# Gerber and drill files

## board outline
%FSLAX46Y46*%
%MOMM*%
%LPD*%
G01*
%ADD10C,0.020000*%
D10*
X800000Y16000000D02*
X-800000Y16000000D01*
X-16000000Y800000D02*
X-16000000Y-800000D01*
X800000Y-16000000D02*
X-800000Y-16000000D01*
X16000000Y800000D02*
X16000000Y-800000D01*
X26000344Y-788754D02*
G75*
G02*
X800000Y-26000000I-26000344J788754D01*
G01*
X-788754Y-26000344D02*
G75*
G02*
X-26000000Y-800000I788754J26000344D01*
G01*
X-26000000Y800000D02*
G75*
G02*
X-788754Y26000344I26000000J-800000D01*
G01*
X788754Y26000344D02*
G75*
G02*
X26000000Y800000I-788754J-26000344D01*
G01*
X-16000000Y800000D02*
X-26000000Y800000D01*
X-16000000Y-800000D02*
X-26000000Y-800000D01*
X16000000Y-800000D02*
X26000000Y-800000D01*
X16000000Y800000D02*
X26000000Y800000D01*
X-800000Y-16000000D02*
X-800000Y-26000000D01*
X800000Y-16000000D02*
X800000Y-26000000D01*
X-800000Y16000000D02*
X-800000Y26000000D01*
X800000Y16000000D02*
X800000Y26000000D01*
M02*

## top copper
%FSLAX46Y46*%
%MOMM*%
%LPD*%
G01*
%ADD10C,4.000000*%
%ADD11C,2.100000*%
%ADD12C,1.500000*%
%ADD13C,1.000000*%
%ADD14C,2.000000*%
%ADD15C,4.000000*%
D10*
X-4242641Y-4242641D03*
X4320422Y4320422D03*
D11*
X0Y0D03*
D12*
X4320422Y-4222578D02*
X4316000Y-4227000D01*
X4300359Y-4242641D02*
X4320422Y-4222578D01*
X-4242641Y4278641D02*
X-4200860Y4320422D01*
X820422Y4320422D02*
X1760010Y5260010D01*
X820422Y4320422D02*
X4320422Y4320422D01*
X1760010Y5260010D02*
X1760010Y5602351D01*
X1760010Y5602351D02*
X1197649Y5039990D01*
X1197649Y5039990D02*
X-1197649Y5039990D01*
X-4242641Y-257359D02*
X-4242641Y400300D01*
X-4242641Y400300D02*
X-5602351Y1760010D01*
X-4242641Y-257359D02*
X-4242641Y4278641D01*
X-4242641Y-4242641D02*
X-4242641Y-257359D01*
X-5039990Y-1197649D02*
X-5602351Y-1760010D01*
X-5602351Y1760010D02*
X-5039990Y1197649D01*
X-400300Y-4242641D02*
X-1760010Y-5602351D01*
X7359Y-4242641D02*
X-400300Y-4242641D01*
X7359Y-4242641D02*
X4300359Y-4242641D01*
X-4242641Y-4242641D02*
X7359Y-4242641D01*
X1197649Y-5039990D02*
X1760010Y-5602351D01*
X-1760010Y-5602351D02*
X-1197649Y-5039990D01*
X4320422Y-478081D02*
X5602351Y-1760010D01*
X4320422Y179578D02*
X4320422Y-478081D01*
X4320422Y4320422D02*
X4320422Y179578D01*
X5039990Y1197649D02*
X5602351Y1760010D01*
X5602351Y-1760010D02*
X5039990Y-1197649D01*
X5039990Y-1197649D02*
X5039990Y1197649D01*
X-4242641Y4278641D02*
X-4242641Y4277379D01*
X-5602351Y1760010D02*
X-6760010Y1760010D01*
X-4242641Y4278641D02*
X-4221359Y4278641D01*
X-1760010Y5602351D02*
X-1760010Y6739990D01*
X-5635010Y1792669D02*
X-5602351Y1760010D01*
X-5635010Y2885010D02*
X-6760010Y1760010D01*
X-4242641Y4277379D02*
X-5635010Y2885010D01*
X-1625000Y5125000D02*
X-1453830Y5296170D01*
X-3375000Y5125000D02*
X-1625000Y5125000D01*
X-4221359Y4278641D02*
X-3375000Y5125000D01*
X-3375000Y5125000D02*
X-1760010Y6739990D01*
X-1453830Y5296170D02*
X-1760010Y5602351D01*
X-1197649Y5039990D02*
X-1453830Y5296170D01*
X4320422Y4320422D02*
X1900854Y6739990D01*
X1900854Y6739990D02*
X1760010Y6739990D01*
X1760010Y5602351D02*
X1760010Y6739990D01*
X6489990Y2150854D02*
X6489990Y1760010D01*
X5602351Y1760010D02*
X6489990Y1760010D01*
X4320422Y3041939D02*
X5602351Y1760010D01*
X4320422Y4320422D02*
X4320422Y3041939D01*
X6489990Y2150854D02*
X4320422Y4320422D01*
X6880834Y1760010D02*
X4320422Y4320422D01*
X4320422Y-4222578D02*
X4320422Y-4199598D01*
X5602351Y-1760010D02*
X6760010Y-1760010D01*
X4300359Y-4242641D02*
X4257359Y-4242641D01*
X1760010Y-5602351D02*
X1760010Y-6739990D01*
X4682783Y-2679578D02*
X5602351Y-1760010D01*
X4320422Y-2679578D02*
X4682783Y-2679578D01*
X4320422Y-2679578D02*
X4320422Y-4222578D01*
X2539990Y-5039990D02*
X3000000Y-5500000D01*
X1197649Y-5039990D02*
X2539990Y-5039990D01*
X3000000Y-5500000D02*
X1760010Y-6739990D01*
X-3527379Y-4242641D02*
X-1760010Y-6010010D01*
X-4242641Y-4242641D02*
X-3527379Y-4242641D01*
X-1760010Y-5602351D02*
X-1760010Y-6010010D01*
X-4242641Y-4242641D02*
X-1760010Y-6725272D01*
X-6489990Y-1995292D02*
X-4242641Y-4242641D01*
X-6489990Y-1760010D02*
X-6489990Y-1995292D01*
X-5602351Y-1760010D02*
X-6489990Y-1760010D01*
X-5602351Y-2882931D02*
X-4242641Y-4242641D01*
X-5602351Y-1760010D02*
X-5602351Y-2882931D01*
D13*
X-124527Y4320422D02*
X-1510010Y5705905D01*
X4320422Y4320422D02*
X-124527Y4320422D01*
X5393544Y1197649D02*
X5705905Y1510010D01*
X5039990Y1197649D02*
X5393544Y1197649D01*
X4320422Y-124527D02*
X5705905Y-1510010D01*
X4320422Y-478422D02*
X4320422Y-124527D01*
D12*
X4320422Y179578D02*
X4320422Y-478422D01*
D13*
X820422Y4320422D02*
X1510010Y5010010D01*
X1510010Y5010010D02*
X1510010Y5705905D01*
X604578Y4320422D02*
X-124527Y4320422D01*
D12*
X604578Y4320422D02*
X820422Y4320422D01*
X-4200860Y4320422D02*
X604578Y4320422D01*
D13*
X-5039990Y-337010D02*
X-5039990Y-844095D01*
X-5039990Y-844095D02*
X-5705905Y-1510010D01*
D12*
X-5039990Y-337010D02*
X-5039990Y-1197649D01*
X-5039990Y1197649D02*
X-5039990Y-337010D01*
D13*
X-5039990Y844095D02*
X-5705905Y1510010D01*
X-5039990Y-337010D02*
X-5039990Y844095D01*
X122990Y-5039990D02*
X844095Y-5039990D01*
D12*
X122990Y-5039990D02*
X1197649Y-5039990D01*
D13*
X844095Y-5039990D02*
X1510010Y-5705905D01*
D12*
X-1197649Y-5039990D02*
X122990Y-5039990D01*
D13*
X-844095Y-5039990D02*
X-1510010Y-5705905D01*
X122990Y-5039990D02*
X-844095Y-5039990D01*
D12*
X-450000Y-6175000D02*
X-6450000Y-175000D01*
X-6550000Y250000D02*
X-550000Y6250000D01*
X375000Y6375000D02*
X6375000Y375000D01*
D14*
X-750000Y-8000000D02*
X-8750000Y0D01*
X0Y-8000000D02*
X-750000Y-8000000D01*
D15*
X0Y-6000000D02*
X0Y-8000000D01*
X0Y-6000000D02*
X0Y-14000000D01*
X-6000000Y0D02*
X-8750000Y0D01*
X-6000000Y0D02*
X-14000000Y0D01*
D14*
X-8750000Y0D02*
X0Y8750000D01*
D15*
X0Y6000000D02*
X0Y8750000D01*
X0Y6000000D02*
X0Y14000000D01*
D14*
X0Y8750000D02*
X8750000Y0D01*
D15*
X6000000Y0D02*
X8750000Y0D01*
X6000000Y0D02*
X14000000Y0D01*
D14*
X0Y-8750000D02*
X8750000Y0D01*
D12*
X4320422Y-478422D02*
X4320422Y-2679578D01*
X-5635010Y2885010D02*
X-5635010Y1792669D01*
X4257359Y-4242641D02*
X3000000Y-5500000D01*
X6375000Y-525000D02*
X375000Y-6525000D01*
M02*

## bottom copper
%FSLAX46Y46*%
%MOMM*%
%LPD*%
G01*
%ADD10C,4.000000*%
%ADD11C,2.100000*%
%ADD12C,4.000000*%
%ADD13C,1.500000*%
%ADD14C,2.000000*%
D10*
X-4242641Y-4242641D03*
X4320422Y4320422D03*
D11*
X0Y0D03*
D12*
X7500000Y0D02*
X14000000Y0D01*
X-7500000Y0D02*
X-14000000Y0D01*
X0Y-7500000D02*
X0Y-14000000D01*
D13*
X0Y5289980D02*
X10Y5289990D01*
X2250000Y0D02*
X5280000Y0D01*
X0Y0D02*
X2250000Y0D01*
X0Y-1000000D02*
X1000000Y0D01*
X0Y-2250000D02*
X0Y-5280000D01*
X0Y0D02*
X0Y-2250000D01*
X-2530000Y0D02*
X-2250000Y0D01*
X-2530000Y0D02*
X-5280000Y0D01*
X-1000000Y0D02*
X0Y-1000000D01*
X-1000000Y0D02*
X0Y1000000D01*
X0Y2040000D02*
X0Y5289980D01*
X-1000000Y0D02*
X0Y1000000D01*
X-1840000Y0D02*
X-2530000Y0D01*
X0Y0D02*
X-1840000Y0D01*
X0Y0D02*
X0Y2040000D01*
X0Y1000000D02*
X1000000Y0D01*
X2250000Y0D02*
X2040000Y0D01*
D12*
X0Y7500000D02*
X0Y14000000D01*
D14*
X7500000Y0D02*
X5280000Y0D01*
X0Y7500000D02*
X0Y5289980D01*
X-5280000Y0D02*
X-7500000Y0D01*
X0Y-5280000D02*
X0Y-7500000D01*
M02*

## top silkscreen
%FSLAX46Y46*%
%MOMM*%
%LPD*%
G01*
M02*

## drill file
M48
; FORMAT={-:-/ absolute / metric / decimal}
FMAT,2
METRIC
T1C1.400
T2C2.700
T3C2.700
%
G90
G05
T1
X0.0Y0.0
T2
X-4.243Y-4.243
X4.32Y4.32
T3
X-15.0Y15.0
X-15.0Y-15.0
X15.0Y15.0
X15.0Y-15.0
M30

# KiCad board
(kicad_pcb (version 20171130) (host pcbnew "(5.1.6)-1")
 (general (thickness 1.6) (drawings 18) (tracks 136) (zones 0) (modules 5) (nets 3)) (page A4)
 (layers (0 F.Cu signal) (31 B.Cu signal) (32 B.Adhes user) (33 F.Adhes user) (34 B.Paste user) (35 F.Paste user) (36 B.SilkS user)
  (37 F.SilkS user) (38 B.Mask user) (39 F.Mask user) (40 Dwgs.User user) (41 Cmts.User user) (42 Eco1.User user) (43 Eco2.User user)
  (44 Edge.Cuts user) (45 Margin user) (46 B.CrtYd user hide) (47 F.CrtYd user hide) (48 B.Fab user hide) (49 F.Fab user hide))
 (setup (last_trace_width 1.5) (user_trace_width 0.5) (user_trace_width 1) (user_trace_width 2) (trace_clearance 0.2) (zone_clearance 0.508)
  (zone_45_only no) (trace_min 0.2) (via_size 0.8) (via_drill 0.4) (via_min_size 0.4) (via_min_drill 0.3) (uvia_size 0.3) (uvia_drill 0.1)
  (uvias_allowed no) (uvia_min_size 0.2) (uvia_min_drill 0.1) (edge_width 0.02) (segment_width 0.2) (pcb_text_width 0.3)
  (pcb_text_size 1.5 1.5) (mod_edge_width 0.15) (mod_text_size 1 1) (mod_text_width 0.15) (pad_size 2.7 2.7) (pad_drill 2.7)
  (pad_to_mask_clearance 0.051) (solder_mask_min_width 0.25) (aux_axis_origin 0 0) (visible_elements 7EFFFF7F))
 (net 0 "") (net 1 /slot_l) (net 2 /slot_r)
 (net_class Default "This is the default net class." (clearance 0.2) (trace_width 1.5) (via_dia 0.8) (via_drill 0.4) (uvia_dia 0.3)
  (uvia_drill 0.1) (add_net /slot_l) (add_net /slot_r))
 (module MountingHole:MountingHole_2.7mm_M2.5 (layer F.Cu) (at -15 -15 90)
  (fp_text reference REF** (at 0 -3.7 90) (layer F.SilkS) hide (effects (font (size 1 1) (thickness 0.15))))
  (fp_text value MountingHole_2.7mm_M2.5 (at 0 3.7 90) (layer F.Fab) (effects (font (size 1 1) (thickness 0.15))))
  (pad 1 np_thru_hole circle (at 0 0 90) (size 2.7 2.7) (drill 2.7) (layers *.Cu *.Mask)))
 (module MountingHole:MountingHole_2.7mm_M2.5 (layer F.Cu) (at 15 -15)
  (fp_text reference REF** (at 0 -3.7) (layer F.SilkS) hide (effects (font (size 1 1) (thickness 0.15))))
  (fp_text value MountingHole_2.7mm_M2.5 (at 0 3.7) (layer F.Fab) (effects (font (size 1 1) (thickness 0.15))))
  (pad 1 np_thru_hole circle (at 0 0) (size 2.7 2.7) (drill 2.7) (layers *.Cu *.Mask)))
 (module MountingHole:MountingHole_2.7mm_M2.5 (layer F.Cu) (at 15 15)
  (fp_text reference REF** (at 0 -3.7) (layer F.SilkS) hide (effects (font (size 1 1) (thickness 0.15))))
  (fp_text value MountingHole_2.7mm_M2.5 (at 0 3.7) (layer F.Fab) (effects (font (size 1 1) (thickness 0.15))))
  (pad 1 np_thru_hole circle (at 0 0) (size 2.7 2.7) (drill 2.7) (layers *.Cu *.Mask)))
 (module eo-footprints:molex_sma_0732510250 (layer F.Cu) (at 0 0 45)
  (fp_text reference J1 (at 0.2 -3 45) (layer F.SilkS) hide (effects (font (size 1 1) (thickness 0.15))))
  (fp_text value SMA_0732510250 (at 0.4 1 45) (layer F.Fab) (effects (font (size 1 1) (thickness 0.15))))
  (pad 2 thru_hole circle (at -6 0 45) (size 4 4) (drill 2.7) (layers *.Cu *.Mask) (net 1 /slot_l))
  (pad 2 thru_hole circle (at 6.11 0 45) (size 4 4) (drill 2.7) (layers *.Cu *.Mask) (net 1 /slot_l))
  (pad 1 thru_hole circle (at 0 0 45) (size 2.1 2.1) (drill 1.4) (layers *.Cu *.Mask) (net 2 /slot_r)))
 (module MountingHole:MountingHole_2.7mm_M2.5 (layer F.Cu) (at -15 15)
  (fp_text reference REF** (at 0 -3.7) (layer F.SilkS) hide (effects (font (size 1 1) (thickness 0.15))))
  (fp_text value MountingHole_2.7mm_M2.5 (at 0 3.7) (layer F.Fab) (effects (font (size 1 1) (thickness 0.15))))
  (pad 1 np_thru_hole circle (at 0 0) (size 2.7 2.7) (drill 2.7) (layers *.Cu *.Mask)))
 (gr_line (start 0.8 -16) (end -0.8 -16) (layer Edge.Cuts) (width 0.02))
 (gr_line (start -16 -0.8) (end -16 0.8) (layer Edge.Cuts) (width 0.02))
 (gr_line (start 0.8 16) (end -0.8 16) (layer Edge.Cuts) (width 0.02))
 (gr_line (start 16 -0.8) (end 16 0.8) (layer Edge.Cuts) (width 0.02))
 (gr_arc (start 0 0) (end 0.8 26) (angle -86.5) (layer Edge.Cuts) (width 0.02))
 (gr_arc (start 0 0) (end -26 0.8) (angle -86.5) (layer Edge.Cuts) (width 0.02))
 (gr_arc (start 0 0) (end -26 -0.8) (angle 86.5) (layer Edge.Cuts) (width 0.02))
 (gr_arc (start 0 0) (end 26 -0.8) (angle -86.5) (layer Edge.Cuts) (width 0.02))
 (gr_line (start -16 -0.8) (end -26 -0.8) (layer Edge.Cuts) (width 0.02))
 (gr_line (start -16 0.8) (end -26 0.8) (layer Edge.Cuts) (width 0.02))
 (gr_line (start 16 0.8) (end 26 0.8) (layer Edge.Cuts) (width 0.02))
 (gr_line (start 16 -0.8) (end 26 -0.8) (layer Edge.Cuts) (width 0.02))
 (gr_line (start -0.8 16) (end -0.8 26) (layer Edge.Cuts) (width 0.02))
 (gr_line (start 0.8 16) (end 0.8 26) (layer Edge.Cuts) (width 0.02))
 (gr_line (start -0.8 -16) (end -0.8 -26) (layer Edge.Cuts) (width 0.02))
 (gr_line (start 0.8 -16) (end 0.8 -26) (layer Edge.Cuts) (width 0.02))
 (segment (start 7.5 0) (end 14 0) (width 4) (layer B.Cu) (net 2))
 (segment (start -7.5 0) (end -14 0) (width 4) (layer B.Cu) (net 2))
 (segment (start 0 7.5) (end 0 14) (width 4) (layer B.Cu) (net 2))
 (segment (start 0 -5.28998) (end 0.00001 -5.28999) (width 1.5) (layer B.Cu) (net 2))
 (segment (start 2.25 0) (end 5.28 0) (width 1.5) (layer B.Cu) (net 2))
 (segment (start 0 0) (end 2.25 0) (width 1.5) (layer B.Cu) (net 2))
 (segment (start 0 1) (end 1 0) (width 1.5) (layer B.Cu) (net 2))
 (segment (start 0 2.25) (end 0 5.28) (width 1.5) (layer B.Cu) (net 2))
 (segment (start 0 0) (end 0 2.25) (width 1.5) (layer B.Cu) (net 2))
 (segment (start -2.53 0) (end -2.25 0) (width 1.5) (layer B.Cu) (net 2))
 (segment (start -2.53 0) (end -5.28 0) (width 1.5) (layer B.Cu) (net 2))
 (segment (start -1 0) (end 0 1) (width 1.5) (layer B.Cu) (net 2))
 (segment (start -1 0) (end 0 -1) (width 1.5) (layer B.Cu) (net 2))
 (segment (start 0 -2.04) (end 0 -5.28998) (width 1.5) (layer B.Cu) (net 2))
 (segment (start -1 0) (end 0 -1) (width 1.5) (layer B.Cu) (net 2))
 (segment (start -1.84 0) (end -2.53 0) (width 1.5) (layer B.Cu) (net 2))
 (segment (start 0 0) (end -1.84 0) (width 1.5) (layer B.Cu) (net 2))
 (segment (start 0 0) (end 0 -2.04) (width 1.5) (layer B.Cu) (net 2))
 (segment (start 0 -1) (end 1 0) (width 1.5) (layer B.Cu) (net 2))
 (segment (start 2.25 0) (end 2.04 0) (width 1.5) (layer B.Cu) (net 2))
 (segment (start 0 -7.5) (end 0 -14) (width 4) (layer B.Cu) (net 2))
 (segment (start 7.5 0) (end 5.28 0) (width 2) (layer B.Cu) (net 2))
 (segment (start 0 -7.5) (end 0 -5.28998) (width 2) (layer B.Cu) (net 2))
 (segment (start -5.28 0) (end -7.5 0) (width 2) (layer B.Cu) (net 2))
 (segment (start 0 5.28) (end 0 7.5) (width 2) (layer B.Cu) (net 2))
 (segment (start 4.320422 4.222578) (end 4.316 4.227) (width 1.5) (layer F.Cu) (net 1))
 (segment (start 4.300359 4.242641) (end 4.320422 4.222578) (width 1.5) (layer F.Cu) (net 1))
 (segment (start -4.242641 -4.278641) (end -4.20086 -4.320422) (width 1.5) (layer F.Cu) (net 1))
 (segment (start 0.820422 -4.320422) (end 1.76001 -5.26001) (width 1.5) (layer F.Cu) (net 1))
 (segment (start 0.820422 -4.320422) (end 4.320422 -4.320422) (width 1.5) (layer F.Cu) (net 1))
 (segment (start 1.76001 -5.26001) (end 1.76001 -5.602351) (width 1.5) (layer F.Cu) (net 1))
 (segment (start 1.76001 -5.602351) (end 1.197649 -5.03999) (width 1.5) (layer F.Cu) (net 1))
 (segment (start 1.197649 -5.03999) (end -1.197649 -5.03999) (width 1.5) (layer F.Cu) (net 1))
 (segment (start -4.242641 0.257359) (end -4.242641 -0.4003) (width 1.5) (layer F.Cu) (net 1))
 (segment (start -4.242641 -0.4003) (end -5.602351 -1.76001) (width 1.5) (layer F.Cu) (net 1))
 (segment (start -4.242641 0.257359) (end -4.242641 -4.278641) (width 1.5) (layer F.Cu) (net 1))
 (segment (start -4.242641 4.242641) (end -4.242641 0.257359) (width 1.5) (layer F.Cu) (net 1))
 (segment (start -5.03999 1.197649) (end -5.602351 1.76001) (width 1.5) (layer F.Cu) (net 1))
 (segment (start -5.602351 -1.76001) (end -5.03999 -1.197649) (width 1.5) (layer F.Cu) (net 1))
 (segment (start -0.4003 4.242641) (end -1.76001 5.602351) (width 1.5) (layer F.Cu) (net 1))
 (segment (start 0.007359 4.242641) (end -0.4003 4.242641) (width 1.5) (layer F.Cu) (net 1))
 (segment (start 0.007359 4.242641) (end 4.300359 4.242641) (width 1.5) (layer F.Cu) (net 1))
 (segment (start -4.242641 4.242641) (end 0.007359 4.242641) (width 1.5) (layer F.Cu) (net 1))
 (segment (start 1.197649 5.03999) (end 1.76001 5.602351) (width 1.5) (layer F.Cu) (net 1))
 (segment (start -1.76001 5.602351) (end -1.197649 5.03999) (width 1.5) (layer F.Cu) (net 1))
 (segment (start 4.320422 0.478081) (end 5.602351 1.76001) (width 1.5) (layer F.Cu) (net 1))
 (segment (start 4.320422 -0.179578) (end 4.320422 0.478081) (width 1.5) (layer F.Cu) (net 1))
 (segment (start 4.320422 -4.320422) (end 4.320422 -0.179578) (width 1.5) (layer F.Cu) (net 1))
 (segment (start 5.03999 -1.197649) (end 5.602351 -1.76001) (width 1.5) (layer F.Cu) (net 1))
 (segment (start 5.602351 1.76001) (end 5.03999 1.197649) (width 1.5) (layer F.Cu) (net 1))
 (segment (start 5.03999 1.197649) (end 5.03999 -1.197649) (width 1.5) (layer F.Cu) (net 1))
 (segment (start -4.242641 -4.278641) (end -4.242641 -4.277379) (width 1.5) (layer F.Cu) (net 1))
 (segment (start -5.602351 -1.76001) (end -6.76001 -1.76001) (width 1.5) (layer F.Cu) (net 1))
 (segment (start -4.242641 -4.278641) (end -4.221359 -4.278641) (width 1.5) (layer F.Cu) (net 1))
 (segment (start -1.76001 -5.602351) (end -1.76001 -6.73999) (width 1.5) (layer F.Cu) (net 1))
 (segment (start -5.63501 -1.792669) (end -5.602351 -1.76001) (width 1.5) (layer F.Cu) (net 1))
 (segment (start -5.63501 -2.88501) (end -6.76001 -1.76001) (width 1.5) (layer F.Cu) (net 1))
 (segment (start -4.242641 -4.277379) (end -5.63501 -2.88501) (width 1.5) (layer F.Cu) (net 1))
 (segment (start -1.625 -5.125) (end -1.45383 -5.29617) (width 1.5) (layer F.Cu) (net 1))
 (segment (start -3.375 -5.125) (end -1.625 -5.125) (width 1.5) (layer F.Cu) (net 1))
 (segment (start -4.221359 -4.278641) (end -3.375 -5.125) (width 1.5) (layer F.Cu) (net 1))
 (segment (start -3.375 -5.125) (end -1.76001 -6.73999) (width 1.5) (layer F.Cu) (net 1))
 (segment (start -1.45383 -5.29617) (end -1.76001 -5.602351) (width 1.5) (layer F.Cu) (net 1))
 (segment (start -1.197649 -5.03999) (end -1.45383 -5.29617) (width 1.5) (layer F.Cu) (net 1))
 (segment (start 4.320422 -4.320422) (end 1.900854 -6.73999) (width 1.5) (layer F.Cu) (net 1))
 (segment (start 1.900854 -6.73999) (end 1.76001 -6.73999) (width 1.5) (layer F.Cu) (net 1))
 (segment (start 1.76001 -5.602351) (end 1.76001 -6.73999) (width 1.5) (layer F.Cu) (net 1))
 (segment (start 6.48999 -2.150854) (end 6.48999 -1.76001) (width 1.5) (layer F.Cu) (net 1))
 (segment (start 5.602351 -1.76001) (end 6.48999 -1.76001) (width 1.5) (layer F.Cu) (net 1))
 (segment (start 4.320422 -3.041939) (end 5.602351 -1.76001) (width 1.5) (layer F.Cu) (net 1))
 (segment (start 4.320422 -4.320422) (end 4.320422 -3.041939) (width 1.5) (layer F.Cu) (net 1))
 (segment (start 6.48999 -2.150854) (end 4.320422 -4.320422) (width 1.5) (layer F.Cu) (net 1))
 (segment (start 6.880834 -1.76001) (end 4.320422 -4.320422) (width 1.5) (layer F.Cu) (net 1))
 (segment (start 4.320422 4.222578) (end 4.320422 4.199598) (width 1.5) (layer F.Cu) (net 1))
 (segment (start 5.602351 1.76001) (end 6.76001 1.76001) (width 1.5) (layer F.Cu) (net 1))
 (segment (start 4.300359 4.242641) (end 4.257359 4.242641) (width 1.5) (layer F.Cu) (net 1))
 (segment (start 1.76001 5.602351) (end 1.76001 6.73999) (width 1.5) (layer F.Cu) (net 1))
 (segment (start 4.682783 2.679578) (end 5.602351 1.76001) (width 1.5) (layer F.Cu) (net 1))
 (segment (start 4.320422 2.679578) (end 4.682783 2.679578) (width 1.5) (layer F.Cu) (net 1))
 (segment (start 4.320422 2.679578) (end 4.320422 4.222578) (width 1.5) (layer F.Cu) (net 1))
 (segment (start 2.53999 5.03999) (end 3 5.5) (width 1.5) (layer F.Cu) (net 1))
 (segment (start 1.197649 5.03999) (end 2.53999 5.03999) (width 1.5) (layer F.Cu) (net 1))
 (segment (start 3 5.5) (end 1.76001 6.73999) (width 1.5) (layer F.Cu) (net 1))
 (segment (start -3.527379 4.242641) (end -1.76001 6.01001) (width 1.5) (layer F.Cu) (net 1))
 (segment (start -4.242641 4.242641) (end -3.527379 4.242641) (width 1.5) (layer F.Cu) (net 1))
 (segment (start -1.76001 5.602351) (end -1.76001 6.01001) (width 1.5) (layer F.Cu) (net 1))
 (segment (start -4.242641 4.242641) (end -1.76001 6.725272) (width 1.5) (layer F.Cu) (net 1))
 (segment (start -6.48999 1.995292) (end -4.242641 4.242641) (width 1.5) (layer F.Cu) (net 1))
 (segment (start -6.48999 1.76001) (end -6.48999 1.995292) (width 1.5) (layer F.Cu) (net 1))
 (segment (start -5.602351 1.76001) (end -6.48999 1.76001) (width 1.5) (layer F.Cu) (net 1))
 (segment (start -5.602351 2.882931) (end -4.242641 4.242641) (width 1.5) (layer F.Cu) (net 1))
 (segment (start -5.602351 1.76001) (end -5.602351 2.882931) (width 1.5) (layer F.Cu) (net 1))
 (segment (start -0.124527 -4.320422) (end -1.51001 -5.705905) (width 1) (layer F.Cu) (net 1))
 (segment (start 4.320422 -4.320422) (end -0.124527 -4.320422) (width 1) (layer F.Cu) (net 1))
 (segment (start 5.393544 -1.197649) (end 5.705905 -1.51001) (width 1) (layer F.Cu) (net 1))
 (segment (start 5.03999 -1.197649) (end 5.393544 -1.197649) (width 1) (layer F.Cu) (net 1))
 (segment (start 4.320422 0.124527) (end 5.705905 1.51001) (width 1) (layer F.Cu) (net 1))
 (segment (start 4.320422 0.478422) (end 4.320422 0.124527) (width 1) (layer F.Cu) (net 1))
 (segment (start 4.320422 -0.179578) (end 4.320422 0.478422) (width 1.5) (layer F.Cu) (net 1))
 (segment (start 0.820422 -4.320422) (end 1.51001 -5.01001) (width 1) (layer F.Cu) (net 1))
 (segment (start 1.51001 -5.01001) (end 1.51001 -5.705905) (width 1) (layer F.Cu) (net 1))
 (segment (start 0.604578 -4.320422) (end -0.124527 -4.320422) (width 1) (layer F.Cu) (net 1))
 (segment (start 0.604578 -4.320422) (end 0.820422 -4.320422) (width 1.5) (layer F.Cu) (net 1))
 (segment (start -4.20086 -4.320422) (end 0.604578 -4.320422) (width 1.5) (layer F.Cu) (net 1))
 (segment (start -5.03999 0.33701) (end -5.03999 0.844095) (width 1) (layer F.Cu) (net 1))
 (segment (start -5.03999 0.844095) (end -5.705905 1.51001) (width 1) (layer F.Cu) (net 1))
 (segment (start -5.03999 0.33701) (end -5.03999 1.197649) (width 1.5) (layer F.Cu) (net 1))
 (segment (start -5.03999 -1.197649) (end -5.03999 0.33701) (width 1.5) (layer F.Cu) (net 1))
 (segment (start -5.03999 -0.844095) (end -5.705905 -1.51001) (width 1) (layer F.Cu) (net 1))
 (segment (start -5.03999 0.33701) (end -5.03999 -0.844095) (width 1) (layer F.Cu) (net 1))
 (segment (start 0.12299 5.03999) (end 0.844095 5.03999) (width 1) (layer F.Cu) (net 1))
 (segment (start 0.12299 5.03999) (end 1.197649 5.03999) (width 1.5) (layer F.Cu) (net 1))
 (segment (start 0.844095 5.03999) (end 1.51001 5.705905) (width 1) (layer F.Cu) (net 1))
 (segment (start -1.197649 5.03999) (end 0.12299 5.03999) (width 1.5) (layer F.Cu) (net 1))
 (segment (start -0.844095 5.03999) (end -1.51001 5.705905) (width 1) (layer F.Cu) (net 1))
 (segment (start 0.12299 5.03999) (end -0.844095 5.03999) (width 1) (layer F.Cu) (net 1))
 (segment (start -0.45 6.175) (end -6.45 0.175) (width 1.5) (layer F.Cu) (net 1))
 (segment (start -6.55 -0.25) (end -0.55 -6.25) (width 1.5) (layer F.Cu) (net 1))
 (segment (start 0.375 -6.375) (end 6.375 -0.375) (width 1.5) (layer F.Cu) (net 1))
 (segment (start -0.75 8) (end -8.75 0) (width 2) (layer F.Cu) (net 1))
 (segment (start 0 8) (end -0.75 8) (width 2) (layer F.Cu) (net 1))
 (segment (start 0 6) (end 0 8) (width 4) (layer F.Cu) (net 1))
 (segment (start 0 6) (end 0 14) (width 4) (layer F.Cu) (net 1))
 (segment (start -6 0) (end -8.75 0) (width 4) (layer F.Cu) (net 1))
 (segment (start -6 0) (end -14 0) (width 4) (layer F.Cu) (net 1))
 (segment (start -8.75 0) (end 0 -8.75) (width 2) (layer F.Cu) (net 1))
 (segment (start 0 -6) (end 0 -8.75) (width 4) (layer F.Cu) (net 1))
 (segment (start 0 -6) (end 0 -14) (width 4) (layer F.Cu) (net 1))
 (segment (start 0 -8.75) (end 8.75 0) (width 2) (layer F.Cu) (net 1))
 (segment (start 6 0) (end 8.75 0) (width 4) (layer F.Cu) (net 1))
 (segment (start 6 0) (end 14 0) (width 4) (layer F.Cu) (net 1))
 (segment (start 0 8.75) (end 8.75 0) (width 2) (layer F.Cu) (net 1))
 (segment (start 4.320422 0.478422) (end 4.320422 2.679578) (width 1.5) (layer F.Cu) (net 1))
 (segment (start -5.63501 -2.88501) (end -5.63501 -1.792669) (width 1.5) (layer F.Cu) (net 1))
 (segment (start 4.257359 4.242641) (end 3 5.5) (width 1.5) (layer F.Cu) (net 1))
 (segment (start 6.375 0.525) (end 0.375 6.525) (width 1.5) (layer F.Cu) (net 1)))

